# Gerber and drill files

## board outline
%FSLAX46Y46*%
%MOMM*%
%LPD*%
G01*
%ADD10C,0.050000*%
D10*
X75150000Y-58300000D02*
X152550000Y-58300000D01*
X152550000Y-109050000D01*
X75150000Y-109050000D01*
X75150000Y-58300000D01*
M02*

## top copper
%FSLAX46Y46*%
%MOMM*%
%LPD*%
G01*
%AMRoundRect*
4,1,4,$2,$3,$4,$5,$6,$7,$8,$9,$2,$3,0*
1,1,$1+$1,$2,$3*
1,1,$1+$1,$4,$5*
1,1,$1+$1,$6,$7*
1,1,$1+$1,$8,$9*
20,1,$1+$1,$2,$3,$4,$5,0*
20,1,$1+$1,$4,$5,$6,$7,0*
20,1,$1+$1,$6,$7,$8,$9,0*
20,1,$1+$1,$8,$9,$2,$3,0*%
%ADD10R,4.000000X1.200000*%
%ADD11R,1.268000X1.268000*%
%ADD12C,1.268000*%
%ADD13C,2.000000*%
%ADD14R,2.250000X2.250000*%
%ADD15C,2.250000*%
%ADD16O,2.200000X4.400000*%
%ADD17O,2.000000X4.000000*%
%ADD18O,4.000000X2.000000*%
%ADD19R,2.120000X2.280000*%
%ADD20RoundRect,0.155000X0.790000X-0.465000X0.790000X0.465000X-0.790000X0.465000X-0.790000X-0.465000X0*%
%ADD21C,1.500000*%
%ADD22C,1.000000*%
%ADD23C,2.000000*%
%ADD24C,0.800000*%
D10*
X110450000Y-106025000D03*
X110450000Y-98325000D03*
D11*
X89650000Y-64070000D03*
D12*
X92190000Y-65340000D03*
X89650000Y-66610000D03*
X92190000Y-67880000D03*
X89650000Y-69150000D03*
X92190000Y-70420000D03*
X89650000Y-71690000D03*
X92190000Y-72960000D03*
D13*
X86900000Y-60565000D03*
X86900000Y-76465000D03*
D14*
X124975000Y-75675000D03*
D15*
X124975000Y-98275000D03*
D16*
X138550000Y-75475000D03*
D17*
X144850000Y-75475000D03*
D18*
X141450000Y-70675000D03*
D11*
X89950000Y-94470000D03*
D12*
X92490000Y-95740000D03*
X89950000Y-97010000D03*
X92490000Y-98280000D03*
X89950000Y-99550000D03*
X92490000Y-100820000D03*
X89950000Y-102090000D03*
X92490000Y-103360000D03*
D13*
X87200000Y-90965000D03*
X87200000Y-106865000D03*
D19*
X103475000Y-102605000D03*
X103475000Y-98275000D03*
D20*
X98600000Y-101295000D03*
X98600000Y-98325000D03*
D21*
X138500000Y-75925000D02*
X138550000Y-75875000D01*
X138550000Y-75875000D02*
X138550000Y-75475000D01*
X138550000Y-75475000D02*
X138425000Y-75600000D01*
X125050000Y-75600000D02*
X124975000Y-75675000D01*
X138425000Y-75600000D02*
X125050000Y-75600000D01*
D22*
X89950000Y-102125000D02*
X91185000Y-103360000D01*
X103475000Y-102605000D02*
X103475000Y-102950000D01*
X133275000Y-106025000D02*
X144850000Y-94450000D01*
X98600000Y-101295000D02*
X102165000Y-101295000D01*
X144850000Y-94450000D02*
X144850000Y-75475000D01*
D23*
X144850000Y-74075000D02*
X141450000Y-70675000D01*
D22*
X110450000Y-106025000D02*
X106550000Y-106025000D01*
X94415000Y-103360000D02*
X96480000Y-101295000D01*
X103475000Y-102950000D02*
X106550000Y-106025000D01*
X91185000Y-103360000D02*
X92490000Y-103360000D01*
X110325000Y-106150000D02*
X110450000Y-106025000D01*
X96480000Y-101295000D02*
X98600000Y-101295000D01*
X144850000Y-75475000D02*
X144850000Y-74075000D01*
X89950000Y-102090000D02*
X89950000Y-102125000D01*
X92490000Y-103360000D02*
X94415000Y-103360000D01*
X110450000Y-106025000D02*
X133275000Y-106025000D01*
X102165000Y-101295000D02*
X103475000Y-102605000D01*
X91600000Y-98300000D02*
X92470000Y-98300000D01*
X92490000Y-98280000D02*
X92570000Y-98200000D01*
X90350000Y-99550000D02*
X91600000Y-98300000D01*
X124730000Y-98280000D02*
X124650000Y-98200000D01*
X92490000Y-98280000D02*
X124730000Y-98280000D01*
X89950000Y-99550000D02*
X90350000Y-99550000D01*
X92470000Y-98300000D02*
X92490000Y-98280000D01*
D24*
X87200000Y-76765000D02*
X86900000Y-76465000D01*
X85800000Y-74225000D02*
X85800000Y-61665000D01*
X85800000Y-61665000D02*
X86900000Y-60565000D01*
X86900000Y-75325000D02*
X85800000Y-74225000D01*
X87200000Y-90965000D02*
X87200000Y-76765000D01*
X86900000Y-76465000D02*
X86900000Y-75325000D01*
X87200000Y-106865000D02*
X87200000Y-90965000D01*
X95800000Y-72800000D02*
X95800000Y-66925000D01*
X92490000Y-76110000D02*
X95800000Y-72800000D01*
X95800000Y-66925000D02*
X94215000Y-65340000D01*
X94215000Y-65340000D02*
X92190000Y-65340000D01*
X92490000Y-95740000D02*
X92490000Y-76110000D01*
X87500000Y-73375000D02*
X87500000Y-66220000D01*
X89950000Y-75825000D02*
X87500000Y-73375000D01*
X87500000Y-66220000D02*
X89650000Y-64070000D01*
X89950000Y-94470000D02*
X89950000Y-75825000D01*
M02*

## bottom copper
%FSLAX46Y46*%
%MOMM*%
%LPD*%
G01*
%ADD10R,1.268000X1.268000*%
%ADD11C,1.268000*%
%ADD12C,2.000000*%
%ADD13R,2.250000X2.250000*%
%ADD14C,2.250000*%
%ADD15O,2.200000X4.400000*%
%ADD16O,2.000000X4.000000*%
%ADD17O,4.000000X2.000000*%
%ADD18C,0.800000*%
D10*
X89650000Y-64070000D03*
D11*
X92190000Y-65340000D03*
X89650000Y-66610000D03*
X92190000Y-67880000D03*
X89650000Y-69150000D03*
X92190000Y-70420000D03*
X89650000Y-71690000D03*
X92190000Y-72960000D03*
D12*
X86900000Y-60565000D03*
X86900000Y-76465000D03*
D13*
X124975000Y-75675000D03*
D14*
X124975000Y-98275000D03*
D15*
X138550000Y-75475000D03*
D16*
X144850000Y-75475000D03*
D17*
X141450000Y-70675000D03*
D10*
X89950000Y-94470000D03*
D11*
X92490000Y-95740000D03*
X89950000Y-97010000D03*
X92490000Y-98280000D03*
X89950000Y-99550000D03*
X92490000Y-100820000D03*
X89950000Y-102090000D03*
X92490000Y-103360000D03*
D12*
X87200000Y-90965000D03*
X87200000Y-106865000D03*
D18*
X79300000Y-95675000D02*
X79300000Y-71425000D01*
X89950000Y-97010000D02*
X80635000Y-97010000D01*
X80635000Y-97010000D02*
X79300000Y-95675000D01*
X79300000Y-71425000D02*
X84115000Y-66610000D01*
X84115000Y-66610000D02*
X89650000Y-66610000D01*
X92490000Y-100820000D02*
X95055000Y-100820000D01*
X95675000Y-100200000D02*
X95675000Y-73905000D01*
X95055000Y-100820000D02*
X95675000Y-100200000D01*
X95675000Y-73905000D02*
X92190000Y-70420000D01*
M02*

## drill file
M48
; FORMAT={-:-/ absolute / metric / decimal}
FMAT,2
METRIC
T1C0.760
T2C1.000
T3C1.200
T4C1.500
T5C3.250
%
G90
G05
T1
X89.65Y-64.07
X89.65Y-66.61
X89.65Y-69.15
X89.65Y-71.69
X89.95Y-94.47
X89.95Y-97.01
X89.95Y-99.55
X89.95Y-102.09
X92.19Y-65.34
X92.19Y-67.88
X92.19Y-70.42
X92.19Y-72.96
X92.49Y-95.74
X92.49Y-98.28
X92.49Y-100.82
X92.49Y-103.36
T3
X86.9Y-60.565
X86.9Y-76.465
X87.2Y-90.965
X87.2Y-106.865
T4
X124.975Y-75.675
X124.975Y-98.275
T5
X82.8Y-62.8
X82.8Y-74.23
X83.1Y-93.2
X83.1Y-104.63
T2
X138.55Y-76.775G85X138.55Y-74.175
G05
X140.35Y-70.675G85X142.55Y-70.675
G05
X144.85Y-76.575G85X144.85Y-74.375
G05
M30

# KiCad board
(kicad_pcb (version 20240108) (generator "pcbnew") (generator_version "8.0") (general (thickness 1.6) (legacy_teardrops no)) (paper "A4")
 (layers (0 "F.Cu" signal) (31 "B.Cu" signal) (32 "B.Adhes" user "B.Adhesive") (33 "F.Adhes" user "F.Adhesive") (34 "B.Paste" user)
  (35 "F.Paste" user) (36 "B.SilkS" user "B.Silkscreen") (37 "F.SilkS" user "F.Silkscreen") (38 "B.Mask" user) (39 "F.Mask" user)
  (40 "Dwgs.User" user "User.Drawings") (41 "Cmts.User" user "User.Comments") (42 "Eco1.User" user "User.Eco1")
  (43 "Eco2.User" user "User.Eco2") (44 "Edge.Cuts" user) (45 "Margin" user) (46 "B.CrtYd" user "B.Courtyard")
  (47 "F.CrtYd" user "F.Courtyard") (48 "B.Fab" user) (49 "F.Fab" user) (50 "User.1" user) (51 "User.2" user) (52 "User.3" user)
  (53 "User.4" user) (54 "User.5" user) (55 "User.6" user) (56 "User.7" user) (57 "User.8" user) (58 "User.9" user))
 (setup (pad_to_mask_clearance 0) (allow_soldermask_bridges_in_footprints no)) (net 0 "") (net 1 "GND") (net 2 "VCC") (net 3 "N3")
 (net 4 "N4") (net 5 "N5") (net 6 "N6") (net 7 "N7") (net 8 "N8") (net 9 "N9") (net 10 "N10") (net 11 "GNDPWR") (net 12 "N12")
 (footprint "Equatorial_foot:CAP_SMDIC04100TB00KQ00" (layer "F.Cu") (at 110.45 102.175 90)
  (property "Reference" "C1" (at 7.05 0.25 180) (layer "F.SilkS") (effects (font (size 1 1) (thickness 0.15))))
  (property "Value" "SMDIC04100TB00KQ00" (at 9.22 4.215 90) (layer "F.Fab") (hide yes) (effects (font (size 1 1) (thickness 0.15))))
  (pad "1" smd rect (at -3.85 0 90) (size 1.2 4) (layers "F.Cu" "F.Paste" "F.Mask") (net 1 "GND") (solder_mask_margin 0.102))
  (pad "2" smd rect (at 3.85 0 90) (size 1.2 4) (layers "F.Cu" "F.Paste" "F.Mask") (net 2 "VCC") (solder_mask_margin 0.102)))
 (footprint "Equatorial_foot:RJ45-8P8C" (layer "F.Cu") (at 83.3 68.515 -90)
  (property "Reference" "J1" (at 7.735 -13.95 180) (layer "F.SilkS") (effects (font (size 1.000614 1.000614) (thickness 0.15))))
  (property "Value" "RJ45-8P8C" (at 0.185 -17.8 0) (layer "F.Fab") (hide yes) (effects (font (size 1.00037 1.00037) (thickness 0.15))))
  (pad "" np_thru_hole circle (at -5.715 0.5 270) (size 3.25 3.25) (drill 3.25) (layers "*.Cu" "*.Mask"))
  (pad "" np_thru_hole circle (at 5.715 0.5 270) (size 3.25 3.25) (drill 3.25) (layers "*.Cu" "*.Mask"))
  (pad "1" thru_hole rect (at -4.445 -6.35 270) (size 1.268 1.268) (drill 0.76) (layers "*.Cu" "*.Mask") (remove_unused_layers no)
   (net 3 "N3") (solder_mask_margin 0.102))
  (pad "2" thru_hole circle (at -3.175 -8.89 270) (size 1.268 1.268) (drill 0.76) (layers "*.Cu" "*.Mask") (remove_unused_layers no)
   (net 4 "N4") (solder_mask_margin 0.102))
  (pad "3" thru_hole circle (at -1.905 -6.35 270) (size 1.268 1.268) (drill 0.76) (layers "*.Cu" "*.Mask") (remove_unused_layers no)
   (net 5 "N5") (solder_mask_margin 0.102))
  (pad "4" thru_hole circle (at -0.635 -8.89 270) (size 1.268 1.268) (drill 0.76) (layers "*.Cu" "*.Mask") (remove_unused_layers no)
   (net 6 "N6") (solder_mask_margin 0.102))
  (pad "5" thru_hole circle (at 0.635 -6.35 270) (size 1.268 1.268) (drill 0.76) (layers "*.Cu" "*.Mask") (remove_unused_layers no)
   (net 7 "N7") (solder_mask_margin 0.102))
  (pad "6" thru_hole circle (at 1.905 -8.89 270) (size 1.268 1.268) (drill 0.76) (layers "*.Cu" "*.Mask") (remove_unused_layers no)
   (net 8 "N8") (solder_mask_margin 0.102))
  (pad "7" thru_hole circle (at 3.175 -6.35 270) (size 1.268 1.268) (drill 0.76) (layers "*.Cu" "*.Mask") (remove_unused_layers no)
   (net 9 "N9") (solder_mask_margin 0.102))
  (pad "8" thru_hole circle (at 4.445 -8.89 270) (size 1.268 1.268) (drill 0.76) (layers "*.Cu" "*.Mask") (remove_unused_layers no)
   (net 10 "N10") (solder_mask_margin 0.102))
  (pad "9" thru_hole circle (at -7.95 -3.6 270) (size 2 2) (drill 1.2) (layers "*.Cu" "*.Mask") (remove_unused_layers no) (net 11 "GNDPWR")
   (solder_mask_margin 0.102))
  (pad "10" thru_hole circle (at 7.95 -3.6 270) (size 2 2) (drill 1.2) (layers "*.Cu" "*.Mask") (remove_unused_layers no) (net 11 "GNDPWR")
   (solder_mask_margin 0.102)))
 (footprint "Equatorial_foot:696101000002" (layer "F.Cu") (at 124.975 75.675 -90)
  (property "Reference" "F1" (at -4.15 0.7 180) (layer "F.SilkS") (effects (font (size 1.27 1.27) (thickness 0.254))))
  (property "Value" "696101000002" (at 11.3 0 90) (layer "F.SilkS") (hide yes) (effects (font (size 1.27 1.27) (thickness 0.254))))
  (pad "1" thru_hole rect (at 0 0 270) (size 2.25 2.25) (drill 1.5) (layers "*.Cu" "*.Mask") (remove_unused_layers no) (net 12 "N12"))
  (pad "2" thru_hole circle (at 22.6 0 270) (size 2.25 2.25) (drill 1.5) (layers "*.Cu" "*.Mask") (remove_unused_layers no) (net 2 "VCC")))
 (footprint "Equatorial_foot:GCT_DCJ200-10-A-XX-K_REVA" (layer "F.Cu") (at 145.1 75.475 90)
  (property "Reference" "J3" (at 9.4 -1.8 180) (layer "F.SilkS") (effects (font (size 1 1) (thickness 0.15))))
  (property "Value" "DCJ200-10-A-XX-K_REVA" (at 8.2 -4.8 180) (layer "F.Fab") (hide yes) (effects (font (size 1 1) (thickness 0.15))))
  (pad "1" thru_hole oval (at 0 -6.55 90) (size 4.4 2.2) (drill oval 3.6 1) (layers "*.Cu" "*.Mask") (remove_unused_layers no)
   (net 12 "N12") (solder_mask_margin 0.102))
  (pad "2" thru_hole oval (at 0 -0.25 90) (size 4 2) (drill oval 3.2 1) (layers "*.Cu" "*.Mask") (remove_unused_layers no) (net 1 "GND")
   (solder_mask_margin 0.102))
  (pad "3" thru_hole oval (at 4.8 -3.65 90) (size 2 4) (drill oval 1 3.2) (layers "*.Cu" "*.Mask") (remove_unused_layers no) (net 1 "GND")
   (solder_mask_margin 0.102)))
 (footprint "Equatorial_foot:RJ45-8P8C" (layer "F.Cu") (at 83.6 98.915 -90)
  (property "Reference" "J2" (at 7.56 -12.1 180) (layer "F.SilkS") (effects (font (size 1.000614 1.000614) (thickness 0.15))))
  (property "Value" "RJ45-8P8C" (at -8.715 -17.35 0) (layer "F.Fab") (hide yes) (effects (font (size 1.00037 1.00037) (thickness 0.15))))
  (pad "" np_thru_hole circle (at -5.715 0.5 270) (size 3.25 3.25) (drill 3.25) (layers "*.Cu" "*.Mask"))
  (pad "" np_thru_hole circle (at 5.715 0.5 270) (size 3.25 3.25) (drill 3.25) (layers "*.Cu" "*.Mask"))
  (pad "1" thru_hole rect (at -4.445 -6.35 270) (size 1.268 1.268) (drill 0.76) (layers "*.Cu" "*.Mask") (remove_unused_layers no)
   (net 3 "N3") (solder_mask_margin 0.102))
  (pad "2" thru_hole circle (at -3.175 -8.89 270) (size 1.268 1.268) (drill 0.76) (layers "*.Cu" "*.Mask") (remove_unused_layers no)
   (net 4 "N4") (solder_mask_margin 0.102))
  (pad "3" thru_hole circle (at -1.905 -6.35 270) (size 1.268 1.268) (drill 0.76) (layers "*.Cu" "*.Mask") (remove_unused_layers no)
   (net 5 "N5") (solder_mask_margin 0.102))
  (pad "4" thru_hole circle (at -0.635 -8.89 270) (size 1.268 1.268) (drill 0.76) (layers "*.Cu" "*.Mask") (remove_unused_layers no)
   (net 2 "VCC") (solder_mask_margin 0.102))
  (pad "5" thru_hole circle (at 0.635 -6.35 270) (size 1.268 1.268) (drill 0.76) (layers "*.Cu" "*.Mask") (remove_unused_layers no)
   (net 2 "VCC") (solder_mask_margin 0.102))
  (pad "6" thru_hole circle (at 1.905 -8.89 270) (size 1.268 1.268) (drill 0.76) (layers "*.Cu" "*.Mask") (remove_unused_layers no)
   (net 8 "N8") (solder_mask_margin 0.102))
  (pad "7" thru_hole circle (at 3.175 -6.35 270) (size 1.268 1.268) (drill 0.76) (layers "*.Cu" "*.Mask") (remove_unused_layers no)
   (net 1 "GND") (solder_mask_margin 0.102))
  (pad "8" thru_hole circle (at 4.445 -8.89 270) (size 1.268 1.268) (drill 0.76) (layers "*.Cu" "*.Mask") (remove_unused_layers no)
   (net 1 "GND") (solder_mask_margin 0.102))
  (pad "9" thru_hole circle (at -7.95 -3.6 270) (size 2 2) (drill 1.2) (layers "*.Cu" "*.Mask") (remove_unused_layers no) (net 11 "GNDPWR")
   (solder_mask_margin 0.102))
  (pad "10" thru_hole circle (at 7.95 -3.6 270) (size 2 2) (drill 1.2) (layers "*.Cu" "*.Mask") (remove_unused_layers no) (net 11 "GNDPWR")
   (solder_mask_margin 0.102)))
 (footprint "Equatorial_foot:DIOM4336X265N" (layer "F.Cu") (at 103.475 100.44 -90)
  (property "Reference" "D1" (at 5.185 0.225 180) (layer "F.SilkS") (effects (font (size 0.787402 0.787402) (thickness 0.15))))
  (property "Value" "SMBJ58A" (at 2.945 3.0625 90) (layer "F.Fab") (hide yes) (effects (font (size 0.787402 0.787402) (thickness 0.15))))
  (pad "A" smd rect (at 2.165 0 270) (size 2.28 2.12) (layers "F.Cu" "F.Paste" "F.Mask") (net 1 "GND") (solder_mask_margin 0.102))
  (pad "C" smd rect (at -2.165 0 270) (size 2.28 2.12) (layers "F.Cu" "F.Paste" "F.Mask") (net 2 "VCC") (solder_mask_margin 0.102)))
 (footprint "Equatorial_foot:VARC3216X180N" (layer "F.Cu") (at 98.6 99.81 90)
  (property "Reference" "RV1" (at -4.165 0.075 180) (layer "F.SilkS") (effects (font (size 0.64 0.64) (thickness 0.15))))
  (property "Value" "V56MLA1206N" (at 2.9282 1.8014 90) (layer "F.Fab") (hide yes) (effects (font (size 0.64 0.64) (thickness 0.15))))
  (pad "1" smd roundrect (at -1.485 0 90) (size 1.24 1.89) (layers "F.Cu" "F.Paste" "F.Mask") (roundrect_rratio 0.125) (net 1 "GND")
   (solder_mask_margin 0.102))
  (pad "2" smd roundrect (at 1.485 0 90) (size 1.24 1.89) (layers "F.Cu" "F.Paste" "F.Mask") (roundrect_rratio 0.125) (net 2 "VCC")
   (solder_mask_margin 0.102)))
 (gr_rect (start 75.15 58.3) (end 152.55 109.05) (stroke (width 0.05) (type default)) (fill none) (layer "Edge.Cuts"))
 (segment (start 138.5 75.925) (end 138.55 75.875) (width 1.5) (layer "F.Cu") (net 12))
 (segment (start 138.55 75.875) (end 138.55 75.475) (width 1.5) (layer "F.Cu") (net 12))
 (segment (start 138.55 75.475) (end 138.425 75.6) (width 1.5) (layer "F.Cu") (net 12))
 (segment (start 125.05 75.6) (end 124.975 75.675) (width 1.5) (layer "F.Cu") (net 12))
 (segment (start 138.425 75.6) (end 125.05 75.6) (width 1.5) (layer "F.Cu") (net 12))
 (segment (start 89.95 102.125) (end 91.185 103.36) (width 1) (layer "F.Cu") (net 1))
 (segment (start 103.475 102.605) (end 103.475 102.95) (width 1) (layer "F.Cu") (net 1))
 (segment (start 133.275 106.025) (end 144.85 94.45) (width 1) (layer "F.Cu") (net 1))
 (segment (start 98.6 101.295) (end 102.165 101.295) (width 1) (layer "F.Cu") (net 1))
 (segment (start 144.85 94.45) (end 144.85 75.475) (width 1) (layer "F.Cu") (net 1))
 (segment (start 144.85 74.075) (end 141.45 70.675) (width 2) (layer "F.Cu") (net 1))
 (segment (start 110.45 106.025) (end 106.55 106.025) (width 1) (layer "F.Cu") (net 1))
 (segment (start 94.415 103.36) (end 96.48 101.295) (width 1) (layer "F.Cu") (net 1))
 (segment (start 103.475 102.95) (end 106.55 106.025) (width 1) (layer "F.Cu") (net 1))
 (segment (start 91.185 103.36) (end 92.49 103.36) (width 1) (layer "F.Cu") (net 1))
 (segment (start 110.325 106.15) (end 110.45 106.025) (width 1) (layer "F.Cu") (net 1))
 (segment (start 96.48 101.295) (end 98.6 101.295) (width 1) (layer "F.Cu") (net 1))
 (segment (start 144.85 75.475) (end 144.85 74.075) (width 1) (layer "F.Cu") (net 1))
 (segment (start 89.95 102.09) (end 89.95 102.125) (width 1) (layer "F.Cu") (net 1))
 (segment (start 92.49 103.36) (end 94.415 103.36) (width 1) (layer "F.Cu") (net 1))
 (segment (start 110.45 106.025) (end 133.275 106.025) (width 1) (layer "F.Cu") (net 1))
 (segment (start 102.165 101.295) (end 103.475 102.605) (width 1) (layer "F.Cu") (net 1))
 (segment (start 91.6 98.3) (end 92.47 98.3) (width 1) (layer "F.Cu") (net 2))
 (segment (start 92.49 98.28) (end 92.57 98.2) (width 1) (layer "F.Cu") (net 2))
 (segment (start 90.35 99.55) (end 91.6 98.3) (width 1) (layer "F.Cu") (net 2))
 (segment (start 124.73 98.28) (end 124.65 98.2) (width 1) (layer "F.Cu") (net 2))
 (segment (start 92.49 98.28) (end 124.73 98.28) (width 1) (layer "F.Cu") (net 2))
 (segment (start 89.95 99.55) (end 90.35 99.55) (width 1) (layer "F.Cu") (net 2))
 (segment (start 92.47 98.3) (end 92.49 98.28) (width 1) (layer "F.Cu") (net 2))
 (segment (start 87.2 76.765) (end 86.9 76.465) (width 0.8) (layer "F.Cu") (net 11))
 (segment (start 85.8 74.225) (end 85.8 61.665) (width 0.8) (layer "F.Cu") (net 11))
 (segment (start 85.8 61.665) (end 86.9 60.565) (width 0.8) (layer "F.Cu") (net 11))
 (segment (start 86.9 75.325) (end 85.8 74.225) (width 0.8) (layer "F.Cu") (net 11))
 (segment (start 87.2 90.965) (end 87.2 76.765) (width 0.8) (layer "F.Cu") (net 11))
 (segment (start 86.9 76.465) (end 86.9 75.325) (width 0.8) (layer "F.Cu") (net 11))
 (segment (start 87.2 106.865) (end 87.2 90.965) (width 0.8) (layer "F.Cu") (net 11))
 (segment (start 95.8 72.8) (end 95.8 66.925) (width 0.8) (layer "F.Cu") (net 4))
 (segment (start 92.49 76.11) (end 95.8 72.8) (width 0.8) (layer "F.Cu") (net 4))
 (segment (start 95.8 66.925) (end 94.215 65.34) (width 0.8) (layer "F.Cu") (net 4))
 (segment (start 94.215 65.34) (end 92.19 65.34) (width 0.8) (layer "F.Cu") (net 4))
 (segment (start 92.49 95.74) (end 92.49 76.11) (width 0.8) (layer "F.Cu") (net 4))
 (segment (start 79.3 95.675) (end 79.3 71.425) (width 0.8) (layer "B.Cu") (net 5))
 (segment (start 89.95 97.01) (end 80.635 97.01) (width 0.8) (layer "B.Cu") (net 5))
 (segment (start 80.635 97.01) (end 79.3 95.675) (width 0.8) (layer "B.Cu") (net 5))
 (segment (start 79.3 71.425) (end 84.115 66.61) (width 0.8) (layer "B.Cu") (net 5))
 (segment (start 84.115 66.61) (end 89.65 66.61) (width 0.8) (layer "B.Cu") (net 5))
 (segment (start 92.49 100.82) (end 95.055 100.82) (width 0.8) (layer "B.Cu") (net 8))
 (segment (start 95.675 100.2) (end 95.675 73.905) (width 0.8) (layer "B.Cu") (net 8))
 (segment (start 95.055 100.82) (end 95.675 100.2) (width 0.8) (layer "B.Cu") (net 8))
 (segment (start 95.675 73.905) (end 92.19 70.42) (width 0.8) (layer "B.Cu") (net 8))
 (segment (start 87.5 73.375) (end 87.5 66.22) (width 0.8) (layer "F.Cu") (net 3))
 (segment (start 89.95 75.825) (end 87.5 73.375) (width 0.8) (layer "F.Cu") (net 3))
 (segment (start 87.5 66.22) (end 89.65 64.07) (width 0.8) (layer "F.Cu") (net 3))
 (segment (start 89.95 94.47) (end 89.95 75.825) (width 0.8) (layer "F.Cu") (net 3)))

